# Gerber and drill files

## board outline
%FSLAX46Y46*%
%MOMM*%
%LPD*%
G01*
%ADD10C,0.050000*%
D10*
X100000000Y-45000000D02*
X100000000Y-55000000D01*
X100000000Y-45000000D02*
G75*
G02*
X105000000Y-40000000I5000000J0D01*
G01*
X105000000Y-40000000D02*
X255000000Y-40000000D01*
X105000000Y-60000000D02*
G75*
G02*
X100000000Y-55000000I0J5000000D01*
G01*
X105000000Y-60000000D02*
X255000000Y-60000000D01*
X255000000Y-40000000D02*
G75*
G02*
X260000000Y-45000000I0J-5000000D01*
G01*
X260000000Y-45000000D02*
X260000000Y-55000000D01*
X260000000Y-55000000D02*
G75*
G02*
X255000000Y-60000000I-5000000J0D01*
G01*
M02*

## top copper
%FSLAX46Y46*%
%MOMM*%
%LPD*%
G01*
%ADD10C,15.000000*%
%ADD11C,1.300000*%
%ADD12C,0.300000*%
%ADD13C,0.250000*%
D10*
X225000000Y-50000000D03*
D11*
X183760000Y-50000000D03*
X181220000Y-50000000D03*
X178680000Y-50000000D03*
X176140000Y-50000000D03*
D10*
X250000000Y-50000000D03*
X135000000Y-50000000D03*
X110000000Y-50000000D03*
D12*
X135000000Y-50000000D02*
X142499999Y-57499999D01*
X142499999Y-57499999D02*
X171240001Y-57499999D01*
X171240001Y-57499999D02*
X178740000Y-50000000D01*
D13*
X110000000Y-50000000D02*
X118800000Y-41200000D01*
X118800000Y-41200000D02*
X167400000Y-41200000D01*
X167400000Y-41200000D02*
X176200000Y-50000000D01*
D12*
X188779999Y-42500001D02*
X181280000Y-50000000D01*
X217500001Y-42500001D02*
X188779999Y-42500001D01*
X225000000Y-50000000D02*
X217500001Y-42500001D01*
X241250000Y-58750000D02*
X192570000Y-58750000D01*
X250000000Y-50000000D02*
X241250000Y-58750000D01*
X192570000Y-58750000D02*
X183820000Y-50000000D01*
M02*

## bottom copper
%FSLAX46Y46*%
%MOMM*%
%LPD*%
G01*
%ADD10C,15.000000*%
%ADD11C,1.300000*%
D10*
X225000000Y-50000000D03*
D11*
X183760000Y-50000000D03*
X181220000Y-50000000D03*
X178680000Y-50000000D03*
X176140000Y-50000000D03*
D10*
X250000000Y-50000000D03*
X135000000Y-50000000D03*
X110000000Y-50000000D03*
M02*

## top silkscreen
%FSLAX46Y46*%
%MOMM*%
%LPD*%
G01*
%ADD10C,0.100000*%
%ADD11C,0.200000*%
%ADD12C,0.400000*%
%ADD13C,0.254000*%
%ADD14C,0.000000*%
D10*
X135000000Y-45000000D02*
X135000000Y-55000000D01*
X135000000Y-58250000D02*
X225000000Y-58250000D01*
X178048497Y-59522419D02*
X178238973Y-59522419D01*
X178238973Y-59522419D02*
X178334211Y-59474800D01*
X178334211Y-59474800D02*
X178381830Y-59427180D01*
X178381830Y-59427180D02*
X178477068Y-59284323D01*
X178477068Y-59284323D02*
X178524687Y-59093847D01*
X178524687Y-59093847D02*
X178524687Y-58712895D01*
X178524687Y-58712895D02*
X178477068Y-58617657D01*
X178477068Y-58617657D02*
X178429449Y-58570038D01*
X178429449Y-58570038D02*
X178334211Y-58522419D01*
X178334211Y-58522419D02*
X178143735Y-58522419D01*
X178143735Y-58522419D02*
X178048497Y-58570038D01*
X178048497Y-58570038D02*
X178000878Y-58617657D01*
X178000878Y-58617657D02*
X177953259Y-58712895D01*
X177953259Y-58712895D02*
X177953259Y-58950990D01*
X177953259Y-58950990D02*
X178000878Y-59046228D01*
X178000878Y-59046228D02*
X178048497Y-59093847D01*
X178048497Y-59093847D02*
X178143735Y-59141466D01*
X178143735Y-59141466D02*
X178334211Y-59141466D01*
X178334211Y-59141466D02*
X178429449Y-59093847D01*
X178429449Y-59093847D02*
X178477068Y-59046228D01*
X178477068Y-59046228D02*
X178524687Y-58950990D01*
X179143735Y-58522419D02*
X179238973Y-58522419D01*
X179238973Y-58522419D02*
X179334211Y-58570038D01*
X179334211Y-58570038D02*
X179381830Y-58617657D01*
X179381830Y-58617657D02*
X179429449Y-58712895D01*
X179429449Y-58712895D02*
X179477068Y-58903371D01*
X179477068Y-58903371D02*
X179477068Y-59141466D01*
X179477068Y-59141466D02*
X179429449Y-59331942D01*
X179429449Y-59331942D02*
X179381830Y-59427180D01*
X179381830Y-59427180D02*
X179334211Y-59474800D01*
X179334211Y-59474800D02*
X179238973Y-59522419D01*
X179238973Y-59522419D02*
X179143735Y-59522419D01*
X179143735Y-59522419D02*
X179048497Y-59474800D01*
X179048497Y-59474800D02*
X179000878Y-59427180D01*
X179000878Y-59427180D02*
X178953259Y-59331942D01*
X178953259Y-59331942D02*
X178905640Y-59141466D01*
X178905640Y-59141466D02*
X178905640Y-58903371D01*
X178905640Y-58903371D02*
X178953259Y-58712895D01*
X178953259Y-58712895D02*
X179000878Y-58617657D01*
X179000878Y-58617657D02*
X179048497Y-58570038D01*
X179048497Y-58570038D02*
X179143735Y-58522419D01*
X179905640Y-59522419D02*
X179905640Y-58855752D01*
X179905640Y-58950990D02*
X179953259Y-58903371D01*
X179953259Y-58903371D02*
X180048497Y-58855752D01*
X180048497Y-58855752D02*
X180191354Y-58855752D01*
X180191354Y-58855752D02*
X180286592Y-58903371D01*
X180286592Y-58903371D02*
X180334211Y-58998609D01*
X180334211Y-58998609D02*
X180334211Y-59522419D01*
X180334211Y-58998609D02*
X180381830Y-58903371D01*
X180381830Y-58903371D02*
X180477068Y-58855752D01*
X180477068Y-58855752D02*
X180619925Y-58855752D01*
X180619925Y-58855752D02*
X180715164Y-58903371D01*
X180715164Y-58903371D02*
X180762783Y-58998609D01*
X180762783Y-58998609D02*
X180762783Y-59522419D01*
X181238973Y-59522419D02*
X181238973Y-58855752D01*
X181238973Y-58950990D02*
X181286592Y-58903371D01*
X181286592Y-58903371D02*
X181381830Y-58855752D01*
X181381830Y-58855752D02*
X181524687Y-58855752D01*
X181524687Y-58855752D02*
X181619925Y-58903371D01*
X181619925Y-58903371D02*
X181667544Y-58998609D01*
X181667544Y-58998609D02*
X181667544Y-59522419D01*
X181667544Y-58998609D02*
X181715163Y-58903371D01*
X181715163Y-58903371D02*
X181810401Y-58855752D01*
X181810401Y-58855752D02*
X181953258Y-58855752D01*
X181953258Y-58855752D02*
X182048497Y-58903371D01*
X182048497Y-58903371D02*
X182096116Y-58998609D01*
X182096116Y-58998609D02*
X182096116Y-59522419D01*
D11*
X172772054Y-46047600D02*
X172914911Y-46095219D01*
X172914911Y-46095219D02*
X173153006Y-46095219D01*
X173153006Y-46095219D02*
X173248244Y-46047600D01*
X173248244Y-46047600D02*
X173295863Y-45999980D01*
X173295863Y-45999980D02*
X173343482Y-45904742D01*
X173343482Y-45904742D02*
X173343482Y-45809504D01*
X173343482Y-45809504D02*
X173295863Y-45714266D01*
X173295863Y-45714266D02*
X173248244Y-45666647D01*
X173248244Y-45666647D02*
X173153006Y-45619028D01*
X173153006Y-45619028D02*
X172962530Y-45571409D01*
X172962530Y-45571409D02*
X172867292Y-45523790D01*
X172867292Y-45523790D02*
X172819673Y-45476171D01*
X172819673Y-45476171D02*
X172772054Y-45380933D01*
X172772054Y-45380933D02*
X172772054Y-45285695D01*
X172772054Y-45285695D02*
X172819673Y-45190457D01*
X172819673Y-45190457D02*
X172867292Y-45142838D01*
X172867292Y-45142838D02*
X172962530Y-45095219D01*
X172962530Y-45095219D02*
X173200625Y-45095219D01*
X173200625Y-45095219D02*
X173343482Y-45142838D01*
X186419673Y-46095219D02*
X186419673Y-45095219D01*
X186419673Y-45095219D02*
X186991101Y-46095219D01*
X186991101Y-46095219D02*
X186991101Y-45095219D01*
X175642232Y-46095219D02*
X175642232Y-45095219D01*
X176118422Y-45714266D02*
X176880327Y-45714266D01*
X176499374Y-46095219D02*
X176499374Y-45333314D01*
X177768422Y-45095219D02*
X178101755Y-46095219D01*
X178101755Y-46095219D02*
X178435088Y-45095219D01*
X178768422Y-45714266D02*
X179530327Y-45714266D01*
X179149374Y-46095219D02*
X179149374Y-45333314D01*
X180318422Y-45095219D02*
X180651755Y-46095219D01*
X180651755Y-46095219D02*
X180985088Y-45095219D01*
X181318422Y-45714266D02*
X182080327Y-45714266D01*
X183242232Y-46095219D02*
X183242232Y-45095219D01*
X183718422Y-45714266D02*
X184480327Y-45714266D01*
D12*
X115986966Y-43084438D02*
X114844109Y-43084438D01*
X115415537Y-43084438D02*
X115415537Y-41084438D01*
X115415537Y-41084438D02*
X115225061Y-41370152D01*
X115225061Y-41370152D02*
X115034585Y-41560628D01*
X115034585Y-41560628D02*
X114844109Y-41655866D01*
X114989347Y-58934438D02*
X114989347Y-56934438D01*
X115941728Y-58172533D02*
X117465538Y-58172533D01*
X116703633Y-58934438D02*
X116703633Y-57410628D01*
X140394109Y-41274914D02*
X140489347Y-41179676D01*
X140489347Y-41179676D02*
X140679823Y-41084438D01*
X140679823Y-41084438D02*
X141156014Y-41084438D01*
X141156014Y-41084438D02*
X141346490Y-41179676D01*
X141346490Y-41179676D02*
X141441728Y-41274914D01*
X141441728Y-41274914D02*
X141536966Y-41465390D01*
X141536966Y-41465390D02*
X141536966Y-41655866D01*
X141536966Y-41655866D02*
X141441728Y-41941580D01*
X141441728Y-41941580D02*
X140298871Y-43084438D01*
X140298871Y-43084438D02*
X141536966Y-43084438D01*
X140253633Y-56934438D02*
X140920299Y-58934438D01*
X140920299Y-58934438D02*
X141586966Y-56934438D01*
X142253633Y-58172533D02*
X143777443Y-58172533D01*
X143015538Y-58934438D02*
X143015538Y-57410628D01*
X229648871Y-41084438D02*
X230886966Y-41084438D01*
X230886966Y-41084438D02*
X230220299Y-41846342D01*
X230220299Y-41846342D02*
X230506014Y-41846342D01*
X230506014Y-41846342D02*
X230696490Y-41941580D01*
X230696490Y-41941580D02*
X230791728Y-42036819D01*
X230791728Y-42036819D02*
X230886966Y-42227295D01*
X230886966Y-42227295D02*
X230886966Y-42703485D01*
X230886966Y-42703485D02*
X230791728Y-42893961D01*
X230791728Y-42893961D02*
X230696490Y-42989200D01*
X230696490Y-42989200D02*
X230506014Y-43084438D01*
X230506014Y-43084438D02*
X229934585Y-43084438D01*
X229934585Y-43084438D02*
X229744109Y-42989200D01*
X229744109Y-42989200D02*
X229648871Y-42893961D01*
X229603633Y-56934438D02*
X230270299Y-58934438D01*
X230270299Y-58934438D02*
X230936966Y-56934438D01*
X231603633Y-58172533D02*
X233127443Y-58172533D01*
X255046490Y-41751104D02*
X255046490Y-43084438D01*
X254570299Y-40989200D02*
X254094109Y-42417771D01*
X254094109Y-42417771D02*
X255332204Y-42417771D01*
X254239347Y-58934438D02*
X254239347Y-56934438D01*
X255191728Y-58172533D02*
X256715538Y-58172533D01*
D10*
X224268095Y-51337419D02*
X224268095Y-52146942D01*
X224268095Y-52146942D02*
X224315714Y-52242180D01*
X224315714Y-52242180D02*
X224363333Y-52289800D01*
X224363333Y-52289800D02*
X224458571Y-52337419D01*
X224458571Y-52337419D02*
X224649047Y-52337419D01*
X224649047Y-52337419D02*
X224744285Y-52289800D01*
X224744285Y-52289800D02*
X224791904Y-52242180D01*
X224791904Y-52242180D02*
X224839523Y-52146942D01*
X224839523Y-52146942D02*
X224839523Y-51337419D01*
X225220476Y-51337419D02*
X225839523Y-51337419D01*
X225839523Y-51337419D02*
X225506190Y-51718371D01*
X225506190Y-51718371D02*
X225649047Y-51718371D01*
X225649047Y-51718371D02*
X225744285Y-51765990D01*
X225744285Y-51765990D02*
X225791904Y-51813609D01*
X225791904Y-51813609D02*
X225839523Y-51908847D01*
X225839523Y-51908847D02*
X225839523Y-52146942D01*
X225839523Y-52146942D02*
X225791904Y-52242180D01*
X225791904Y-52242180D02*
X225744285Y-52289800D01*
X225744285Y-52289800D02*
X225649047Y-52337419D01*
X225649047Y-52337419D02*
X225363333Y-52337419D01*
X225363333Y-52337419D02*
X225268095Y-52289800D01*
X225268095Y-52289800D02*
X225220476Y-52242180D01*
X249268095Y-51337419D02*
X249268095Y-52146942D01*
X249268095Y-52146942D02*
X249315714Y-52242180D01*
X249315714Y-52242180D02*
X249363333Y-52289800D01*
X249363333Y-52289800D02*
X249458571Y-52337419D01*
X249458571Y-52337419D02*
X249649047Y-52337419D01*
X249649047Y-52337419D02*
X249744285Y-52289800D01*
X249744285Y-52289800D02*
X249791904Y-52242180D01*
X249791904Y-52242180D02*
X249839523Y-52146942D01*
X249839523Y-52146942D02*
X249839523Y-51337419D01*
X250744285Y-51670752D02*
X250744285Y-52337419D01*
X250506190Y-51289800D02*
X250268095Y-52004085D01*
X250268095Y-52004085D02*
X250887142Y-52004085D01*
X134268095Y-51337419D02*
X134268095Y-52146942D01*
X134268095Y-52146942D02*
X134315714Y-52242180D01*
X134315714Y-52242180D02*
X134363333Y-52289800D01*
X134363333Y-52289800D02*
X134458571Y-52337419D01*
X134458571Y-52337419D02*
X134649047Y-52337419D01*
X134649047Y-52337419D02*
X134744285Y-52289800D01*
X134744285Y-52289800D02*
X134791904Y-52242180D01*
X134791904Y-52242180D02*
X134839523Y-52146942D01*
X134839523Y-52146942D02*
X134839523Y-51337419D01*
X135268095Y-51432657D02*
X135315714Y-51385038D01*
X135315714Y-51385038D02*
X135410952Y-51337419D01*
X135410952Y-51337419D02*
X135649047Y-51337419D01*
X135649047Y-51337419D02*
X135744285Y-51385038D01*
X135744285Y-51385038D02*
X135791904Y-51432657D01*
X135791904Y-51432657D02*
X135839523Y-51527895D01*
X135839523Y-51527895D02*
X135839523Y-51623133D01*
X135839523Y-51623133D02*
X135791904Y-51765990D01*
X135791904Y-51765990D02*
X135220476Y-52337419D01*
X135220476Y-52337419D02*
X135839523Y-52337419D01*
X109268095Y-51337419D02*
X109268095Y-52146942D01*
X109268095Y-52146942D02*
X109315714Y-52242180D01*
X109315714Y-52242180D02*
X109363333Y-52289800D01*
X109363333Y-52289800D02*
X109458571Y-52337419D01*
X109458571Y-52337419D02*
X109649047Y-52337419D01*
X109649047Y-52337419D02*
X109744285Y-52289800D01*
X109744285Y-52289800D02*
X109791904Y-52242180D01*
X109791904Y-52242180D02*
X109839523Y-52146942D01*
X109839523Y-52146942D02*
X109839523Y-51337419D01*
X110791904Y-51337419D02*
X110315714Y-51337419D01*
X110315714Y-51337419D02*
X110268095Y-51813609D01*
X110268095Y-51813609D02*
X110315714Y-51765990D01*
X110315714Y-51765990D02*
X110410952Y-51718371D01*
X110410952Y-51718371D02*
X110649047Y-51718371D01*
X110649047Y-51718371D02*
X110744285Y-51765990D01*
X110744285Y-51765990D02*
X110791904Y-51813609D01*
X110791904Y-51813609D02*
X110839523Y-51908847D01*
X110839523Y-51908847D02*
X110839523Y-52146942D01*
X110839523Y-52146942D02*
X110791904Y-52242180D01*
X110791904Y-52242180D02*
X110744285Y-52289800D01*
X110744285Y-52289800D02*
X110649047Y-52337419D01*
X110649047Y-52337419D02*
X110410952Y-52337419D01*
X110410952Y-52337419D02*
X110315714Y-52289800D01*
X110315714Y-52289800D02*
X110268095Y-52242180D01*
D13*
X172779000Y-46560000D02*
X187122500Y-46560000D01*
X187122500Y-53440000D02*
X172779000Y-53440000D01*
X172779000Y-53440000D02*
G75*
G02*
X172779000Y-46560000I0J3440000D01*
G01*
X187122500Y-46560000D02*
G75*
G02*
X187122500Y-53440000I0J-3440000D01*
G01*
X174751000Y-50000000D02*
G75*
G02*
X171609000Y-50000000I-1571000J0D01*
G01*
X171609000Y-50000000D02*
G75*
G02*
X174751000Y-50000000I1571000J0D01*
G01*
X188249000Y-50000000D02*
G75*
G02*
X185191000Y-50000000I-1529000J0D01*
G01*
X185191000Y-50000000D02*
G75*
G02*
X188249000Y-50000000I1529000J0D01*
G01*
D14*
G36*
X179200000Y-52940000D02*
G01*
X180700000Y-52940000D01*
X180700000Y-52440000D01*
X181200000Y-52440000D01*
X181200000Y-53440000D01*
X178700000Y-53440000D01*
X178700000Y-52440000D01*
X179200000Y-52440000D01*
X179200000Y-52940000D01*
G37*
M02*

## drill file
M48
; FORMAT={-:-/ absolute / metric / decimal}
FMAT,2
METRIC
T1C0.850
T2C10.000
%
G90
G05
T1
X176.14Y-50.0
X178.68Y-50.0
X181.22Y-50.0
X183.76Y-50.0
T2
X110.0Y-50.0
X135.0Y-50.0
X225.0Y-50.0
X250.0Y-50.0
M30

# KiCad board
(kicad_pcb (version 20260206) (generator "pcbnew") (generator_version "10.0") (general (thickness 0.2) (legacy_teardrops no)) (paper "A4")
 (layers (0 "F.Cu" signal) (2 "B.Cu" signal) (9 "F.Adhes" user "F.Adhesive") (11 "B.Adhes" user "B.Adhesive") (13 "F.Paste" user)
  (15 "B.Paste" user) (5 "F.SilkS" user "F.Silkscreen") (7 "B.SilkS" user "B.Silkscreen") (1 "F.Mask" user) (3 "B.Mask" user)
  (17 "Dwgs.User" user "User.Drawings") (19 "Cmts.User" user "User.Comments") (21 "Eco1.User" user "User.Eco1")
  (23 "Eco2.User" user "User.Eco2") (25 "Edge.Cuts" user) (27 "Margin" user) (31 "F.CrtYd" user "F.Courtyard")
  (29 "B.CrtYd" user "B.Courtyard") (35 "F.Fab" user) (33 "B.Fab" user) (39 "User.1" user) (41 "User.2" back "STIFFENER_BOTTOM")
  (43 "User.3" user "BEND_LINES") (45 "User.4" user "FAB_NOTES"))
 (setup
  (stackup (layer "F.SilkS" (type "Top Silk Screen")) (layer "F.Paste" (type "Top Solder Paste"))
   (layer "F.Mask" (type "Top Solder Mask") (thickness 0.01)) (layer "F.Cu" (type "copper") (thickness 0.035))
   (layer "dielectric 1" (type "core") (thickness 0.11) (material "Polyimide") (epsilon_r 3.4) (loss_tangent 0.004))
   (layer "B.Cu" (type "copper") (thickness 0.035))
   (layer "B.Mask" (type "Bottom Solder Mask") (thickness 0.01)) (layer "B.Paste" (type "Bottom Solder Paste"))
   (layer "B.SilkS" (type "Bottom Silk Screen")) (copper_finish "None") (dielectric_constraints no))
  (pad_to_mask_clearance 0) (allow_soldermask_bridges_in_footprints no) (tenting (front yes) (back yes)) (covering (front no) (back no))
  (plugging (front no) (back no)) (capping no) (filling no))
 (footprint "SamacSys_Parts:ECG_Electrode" (layer "F.Cu") (at 225.03 52.38)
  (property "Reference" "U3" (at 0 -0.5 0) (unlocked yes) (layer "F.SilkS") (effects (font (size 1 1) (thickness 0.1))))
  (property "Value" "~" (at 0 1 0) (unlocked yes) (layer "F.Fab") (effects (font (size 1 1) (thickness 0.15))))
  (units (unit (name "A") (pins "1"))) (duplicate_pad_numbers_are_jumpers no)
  (pad "1" thru_hole circle (at -0.03 -2.38) (size 15 15) (drill 10) (layers "*.Cu" "*.Mask") (remove_unused_layers no) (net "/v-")))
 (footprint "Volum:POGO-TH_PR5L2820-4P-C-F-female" (layer "F.Cu") (at 179.95 50 180)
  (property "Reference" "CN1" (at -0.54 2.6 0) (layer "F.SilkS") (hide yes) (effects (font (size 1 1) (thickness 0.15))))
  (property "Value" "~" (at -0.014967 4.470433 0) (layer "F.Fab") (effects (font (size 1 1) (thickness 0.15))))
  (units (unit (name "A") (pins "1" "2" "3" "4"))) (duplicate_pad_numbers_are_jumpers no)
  (fp_line (start 7.171 3.44) (end -7.1725 3.44) (stroke (width 0.254) (type default)) (layer "F.SilkS"))
  (fp_line (start -7.1725 -3.44) (end 7.171 -3.44) (stroke (width 0.254) (type default)) (layer "F.SilkS"))
  (fp_arc (start 7.171 -3.44) (mid 10.611 0) (end 7.171 3.44) (stroke (width 0.254) (type default)) (layer "F.SilkS"))
  (fp_arc (start -7.1725 3.44) (mid -10.6125 0) (end -7.1725 -3.44) (stroke (width 0.254) (type default)) (layer "F.SilkS"))
  (fp_circle (center 6.77 0) (end 8.341 0) (stroke (width 0.254) (type default)) (fill no) (layer "F.SilkS"))
  (fp_circle (center -6.77 0) (end -5.241 0) (stroke (width 0.254) (type default)) (fill no) (layer "F.SilkS"))
  (fp_poly
   (pts (xy 1.25 -2.44) (xy 1.25 -3.44) (xy -1.25 -3.44) (xy -1.25 -2.44) (xy -0.75 -2.44) (xy -0.75 -2.94) (xy 0.75 -2.94) (xy 0.75 -2.44))
   (stroke (width 0) (type default)) (fill yes) (layer "F.SilkS"))
  (pad "1" thru_hole circle (at -3.81 0 180) (size 1.3 1.3) (drill 0.85) (layers "*.Cu" "*.Mask") (remove_unused_layers no) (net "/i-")
   (thermal_bridge_angle 90))
  (pad "2" thru_hole circle (at -1.27 0 180) (size 1.3 1.3) (drill 0.85) (layers "*.Cu" "*.Mask") (remove_unused_layers no) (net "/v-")
   (thermal_bridge_angle 90))
  (pad "3" thru_hole circle (at 1.27 0 180) (size 1.3 1.3) (drill 0.85) (layers "*.Cu" "*.Mask") (remove_unused_layers no) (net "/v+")
   (thermal_bridge_angle 90))
  (pad "4" thru_hole circle (at 3.81 0 180) (size 1.3 1.3) (drill 0.85) (layers "*.Cu" "*.Mask") (remove_unused_layers no) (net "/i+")
   (thermal_bridge_angle 90)))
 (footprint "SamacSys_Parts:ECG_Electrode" (layer "F.Cu") (at 250.03 52.38)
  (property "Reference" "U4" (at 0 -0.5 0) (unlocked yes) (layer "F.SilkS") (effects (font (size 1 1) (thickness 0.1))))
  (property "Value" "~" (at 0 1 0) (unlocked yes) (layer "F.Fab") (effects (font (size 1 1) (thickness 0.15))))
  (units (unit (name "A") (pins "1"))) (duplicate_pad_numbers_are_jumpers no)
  (pad "1" thru_hole circle (at -0.03 -2.38) (size 15 15) (drill 10) (layers "*.Cu" "*.Mask") (remove_unused_layers no) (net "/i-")))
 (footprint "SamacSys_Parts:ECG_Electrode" (layer "F.Cu") (at 135.03 52.38)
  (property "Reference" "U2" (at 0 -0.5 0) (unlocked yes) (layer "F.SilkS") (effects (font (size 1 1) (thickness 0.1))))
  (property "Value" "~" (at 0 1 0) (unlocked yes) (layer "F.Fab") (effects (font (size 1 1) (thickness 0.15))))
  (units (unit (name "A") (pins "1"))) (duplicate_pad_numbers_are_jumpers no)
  (pad "1" thru_hole circle (at -0.03 -2.38) (size 15 15) (drill 10) (layers "*.Cu" "*.Mask") (remove_unused_layers no) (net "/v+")))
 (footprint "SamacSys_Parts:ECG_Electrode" (layer "F.Cu") (at 110.03 52.38)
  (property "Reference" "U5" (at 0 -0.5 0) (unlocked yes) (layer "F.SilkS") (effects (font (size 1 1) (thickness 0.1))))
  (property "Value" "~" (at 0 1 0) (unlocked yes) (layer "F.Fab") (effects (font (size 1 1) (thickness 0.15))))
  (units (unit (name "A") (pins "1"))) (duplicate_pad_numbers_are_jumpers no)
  (pad "1" thru_hole circle (at -0.03 -2.38) (size 15 15) (drill 10) (layers "*.Cu" "*.Mask") (remove_unused_layers no) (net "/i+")))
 (gr_line (start 135 45) (end 135 55) (stroke (width 0.1) (type default)) (layer "F.SilkS"))
 (gr_line (start 135 58.25) (end 225 58.25) (stroke (width 0.1) (type default)) (layer "F.SilkS"))
 (gr_line (start 100 45) (end 100 55) (stroke (width 0.05) (type default)) (layer "Edge.Cuts"))
 (gr_arc (start 100 45) (mid 101.464466 41.464466) (end 105 40) (stroke (width 0.05) (type default)) (layer "Edge.Cuts"))
 (gr_line (start 105 40) (end 255 40) (stroke (width 0.05) (type default)) (layer "Edge.Cuts"))
 (gr_arc (start 105 60) (mid 101.464466 58.535534) (end 100 55) (stroke (width 0.05) (type default)) (layer "Edge.Cuts"))
 (gr_line (start 105 60) (end 255 60) (stroke (width 0.05) (type default)) (layer "Edge.Cuts"))
 (gr_arc (start 255 40) (mid 258.535534 41.464466) (end 260 45) (stroke (width 0.05) (type default)) (layer "Edge.Cuts"))
 (gr_line (start 260 45) (end 260 55) (stroke (width 0.05) (type default)) (layer "Edge.Cuts"))
 (gr_arc (start 260 55) (mid 258.535534 58.535534) (end 255 60) (stroke (width 0.05) (type default)) (layer "Edge.Cuts"))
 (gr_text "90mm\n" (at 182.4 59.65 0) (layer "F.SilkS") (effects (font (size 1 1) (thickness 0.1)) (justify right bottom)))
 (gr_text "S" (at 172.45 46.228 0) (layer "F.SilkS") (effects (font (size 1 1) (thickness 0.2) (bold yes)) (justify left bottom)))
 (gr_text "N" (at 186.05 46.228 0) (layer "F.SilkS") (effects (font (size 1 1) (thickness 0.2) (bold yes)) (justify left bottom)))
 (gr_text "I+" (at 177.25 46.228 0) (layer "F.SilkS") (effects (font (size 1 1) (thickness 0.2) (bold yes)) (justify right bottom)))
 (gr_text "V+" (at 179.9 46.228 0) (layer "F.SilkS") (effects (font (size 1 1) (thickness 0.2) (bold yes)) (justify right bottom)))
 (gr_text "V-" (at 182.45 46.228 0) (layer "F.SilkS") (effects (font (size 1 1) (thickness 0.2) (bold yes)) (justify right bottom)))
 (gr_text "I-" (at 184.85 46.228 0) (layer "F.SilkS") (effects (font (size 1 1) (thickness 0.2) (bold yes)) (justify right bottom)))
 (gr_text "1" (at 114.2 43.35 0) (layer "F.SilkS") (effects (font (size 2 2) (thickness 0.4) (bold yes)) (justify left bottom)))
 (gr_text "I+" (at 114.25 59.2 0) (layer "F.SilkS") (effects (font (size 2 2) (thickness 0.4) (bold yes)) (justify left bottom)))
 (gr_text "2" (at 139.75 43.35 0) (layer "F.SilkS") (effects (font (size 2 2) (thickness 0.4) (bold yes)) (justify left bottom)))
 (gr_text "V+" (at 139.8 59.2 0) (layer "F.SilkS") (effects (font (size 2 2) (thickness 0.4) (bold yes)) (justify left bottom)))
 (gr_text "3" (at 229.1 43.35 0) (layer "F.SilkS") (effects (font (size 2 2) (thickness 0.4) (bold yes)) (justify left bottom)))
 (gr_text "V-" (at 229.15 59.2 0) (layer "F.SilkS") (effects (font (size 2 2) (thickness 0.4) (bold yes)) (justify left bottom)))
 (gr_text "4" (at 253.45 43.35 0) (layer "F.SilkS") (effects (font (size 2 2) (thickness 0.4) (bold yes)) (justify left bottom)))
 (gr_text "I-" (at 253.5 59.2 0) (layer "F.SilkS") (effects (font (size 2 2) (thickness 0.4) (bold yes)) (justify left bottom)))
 (segment (start 135 50) (end 142.499999 57.499999) (width 0.3) (layer "F.Cu") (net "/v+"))
 (segment (start 142.499999 57.499999) (end 171.240001 57.499999) (width 0.3) (layer "F.Cu") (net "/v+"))
 (segment (start 171.240001 57.499999) (end 178.74 50) (width 0.3) (layer "F.Cu") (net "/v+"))
 (segment (start 110 50) (end 118.8 41.2) (width 0.25) (layer "F.Cu") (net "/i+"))
 (segment (start 118.8 41.2) (end 167.4 41.2) (width 0.25) (layer "F.Cu") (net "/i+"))
 (segment (start 167.4 41.2) (end 176.2 50) (width 0.25) (layer "F.Cu") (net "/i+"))
 (segment (start 188.779999 42.500001) (end 181.28 50) (width 0.3) (layer "F.Cu") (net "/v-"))
 (segment (start 217.500001 42.500001) (end 188.779999 42.500001) (width 0.3) (layer "F.Cu") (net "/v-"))
 (segment (start 225 50) (end 217.500001 42.500001) (width 0.3) (layer "F.Cu") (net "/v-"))
 (segment (start 241.25 58.75) (end 192.57 58.75) (width 0.3) (layer "F.Cu") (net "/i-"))
 (segment (start 250 50) (end 241.25 58.75) (width 0.3) (layer "F.Cu") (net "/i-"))
 (segment (start 192.57 58.75) (end 183.82 50) (width 0.3) (layer "F.Cu") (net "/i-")))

